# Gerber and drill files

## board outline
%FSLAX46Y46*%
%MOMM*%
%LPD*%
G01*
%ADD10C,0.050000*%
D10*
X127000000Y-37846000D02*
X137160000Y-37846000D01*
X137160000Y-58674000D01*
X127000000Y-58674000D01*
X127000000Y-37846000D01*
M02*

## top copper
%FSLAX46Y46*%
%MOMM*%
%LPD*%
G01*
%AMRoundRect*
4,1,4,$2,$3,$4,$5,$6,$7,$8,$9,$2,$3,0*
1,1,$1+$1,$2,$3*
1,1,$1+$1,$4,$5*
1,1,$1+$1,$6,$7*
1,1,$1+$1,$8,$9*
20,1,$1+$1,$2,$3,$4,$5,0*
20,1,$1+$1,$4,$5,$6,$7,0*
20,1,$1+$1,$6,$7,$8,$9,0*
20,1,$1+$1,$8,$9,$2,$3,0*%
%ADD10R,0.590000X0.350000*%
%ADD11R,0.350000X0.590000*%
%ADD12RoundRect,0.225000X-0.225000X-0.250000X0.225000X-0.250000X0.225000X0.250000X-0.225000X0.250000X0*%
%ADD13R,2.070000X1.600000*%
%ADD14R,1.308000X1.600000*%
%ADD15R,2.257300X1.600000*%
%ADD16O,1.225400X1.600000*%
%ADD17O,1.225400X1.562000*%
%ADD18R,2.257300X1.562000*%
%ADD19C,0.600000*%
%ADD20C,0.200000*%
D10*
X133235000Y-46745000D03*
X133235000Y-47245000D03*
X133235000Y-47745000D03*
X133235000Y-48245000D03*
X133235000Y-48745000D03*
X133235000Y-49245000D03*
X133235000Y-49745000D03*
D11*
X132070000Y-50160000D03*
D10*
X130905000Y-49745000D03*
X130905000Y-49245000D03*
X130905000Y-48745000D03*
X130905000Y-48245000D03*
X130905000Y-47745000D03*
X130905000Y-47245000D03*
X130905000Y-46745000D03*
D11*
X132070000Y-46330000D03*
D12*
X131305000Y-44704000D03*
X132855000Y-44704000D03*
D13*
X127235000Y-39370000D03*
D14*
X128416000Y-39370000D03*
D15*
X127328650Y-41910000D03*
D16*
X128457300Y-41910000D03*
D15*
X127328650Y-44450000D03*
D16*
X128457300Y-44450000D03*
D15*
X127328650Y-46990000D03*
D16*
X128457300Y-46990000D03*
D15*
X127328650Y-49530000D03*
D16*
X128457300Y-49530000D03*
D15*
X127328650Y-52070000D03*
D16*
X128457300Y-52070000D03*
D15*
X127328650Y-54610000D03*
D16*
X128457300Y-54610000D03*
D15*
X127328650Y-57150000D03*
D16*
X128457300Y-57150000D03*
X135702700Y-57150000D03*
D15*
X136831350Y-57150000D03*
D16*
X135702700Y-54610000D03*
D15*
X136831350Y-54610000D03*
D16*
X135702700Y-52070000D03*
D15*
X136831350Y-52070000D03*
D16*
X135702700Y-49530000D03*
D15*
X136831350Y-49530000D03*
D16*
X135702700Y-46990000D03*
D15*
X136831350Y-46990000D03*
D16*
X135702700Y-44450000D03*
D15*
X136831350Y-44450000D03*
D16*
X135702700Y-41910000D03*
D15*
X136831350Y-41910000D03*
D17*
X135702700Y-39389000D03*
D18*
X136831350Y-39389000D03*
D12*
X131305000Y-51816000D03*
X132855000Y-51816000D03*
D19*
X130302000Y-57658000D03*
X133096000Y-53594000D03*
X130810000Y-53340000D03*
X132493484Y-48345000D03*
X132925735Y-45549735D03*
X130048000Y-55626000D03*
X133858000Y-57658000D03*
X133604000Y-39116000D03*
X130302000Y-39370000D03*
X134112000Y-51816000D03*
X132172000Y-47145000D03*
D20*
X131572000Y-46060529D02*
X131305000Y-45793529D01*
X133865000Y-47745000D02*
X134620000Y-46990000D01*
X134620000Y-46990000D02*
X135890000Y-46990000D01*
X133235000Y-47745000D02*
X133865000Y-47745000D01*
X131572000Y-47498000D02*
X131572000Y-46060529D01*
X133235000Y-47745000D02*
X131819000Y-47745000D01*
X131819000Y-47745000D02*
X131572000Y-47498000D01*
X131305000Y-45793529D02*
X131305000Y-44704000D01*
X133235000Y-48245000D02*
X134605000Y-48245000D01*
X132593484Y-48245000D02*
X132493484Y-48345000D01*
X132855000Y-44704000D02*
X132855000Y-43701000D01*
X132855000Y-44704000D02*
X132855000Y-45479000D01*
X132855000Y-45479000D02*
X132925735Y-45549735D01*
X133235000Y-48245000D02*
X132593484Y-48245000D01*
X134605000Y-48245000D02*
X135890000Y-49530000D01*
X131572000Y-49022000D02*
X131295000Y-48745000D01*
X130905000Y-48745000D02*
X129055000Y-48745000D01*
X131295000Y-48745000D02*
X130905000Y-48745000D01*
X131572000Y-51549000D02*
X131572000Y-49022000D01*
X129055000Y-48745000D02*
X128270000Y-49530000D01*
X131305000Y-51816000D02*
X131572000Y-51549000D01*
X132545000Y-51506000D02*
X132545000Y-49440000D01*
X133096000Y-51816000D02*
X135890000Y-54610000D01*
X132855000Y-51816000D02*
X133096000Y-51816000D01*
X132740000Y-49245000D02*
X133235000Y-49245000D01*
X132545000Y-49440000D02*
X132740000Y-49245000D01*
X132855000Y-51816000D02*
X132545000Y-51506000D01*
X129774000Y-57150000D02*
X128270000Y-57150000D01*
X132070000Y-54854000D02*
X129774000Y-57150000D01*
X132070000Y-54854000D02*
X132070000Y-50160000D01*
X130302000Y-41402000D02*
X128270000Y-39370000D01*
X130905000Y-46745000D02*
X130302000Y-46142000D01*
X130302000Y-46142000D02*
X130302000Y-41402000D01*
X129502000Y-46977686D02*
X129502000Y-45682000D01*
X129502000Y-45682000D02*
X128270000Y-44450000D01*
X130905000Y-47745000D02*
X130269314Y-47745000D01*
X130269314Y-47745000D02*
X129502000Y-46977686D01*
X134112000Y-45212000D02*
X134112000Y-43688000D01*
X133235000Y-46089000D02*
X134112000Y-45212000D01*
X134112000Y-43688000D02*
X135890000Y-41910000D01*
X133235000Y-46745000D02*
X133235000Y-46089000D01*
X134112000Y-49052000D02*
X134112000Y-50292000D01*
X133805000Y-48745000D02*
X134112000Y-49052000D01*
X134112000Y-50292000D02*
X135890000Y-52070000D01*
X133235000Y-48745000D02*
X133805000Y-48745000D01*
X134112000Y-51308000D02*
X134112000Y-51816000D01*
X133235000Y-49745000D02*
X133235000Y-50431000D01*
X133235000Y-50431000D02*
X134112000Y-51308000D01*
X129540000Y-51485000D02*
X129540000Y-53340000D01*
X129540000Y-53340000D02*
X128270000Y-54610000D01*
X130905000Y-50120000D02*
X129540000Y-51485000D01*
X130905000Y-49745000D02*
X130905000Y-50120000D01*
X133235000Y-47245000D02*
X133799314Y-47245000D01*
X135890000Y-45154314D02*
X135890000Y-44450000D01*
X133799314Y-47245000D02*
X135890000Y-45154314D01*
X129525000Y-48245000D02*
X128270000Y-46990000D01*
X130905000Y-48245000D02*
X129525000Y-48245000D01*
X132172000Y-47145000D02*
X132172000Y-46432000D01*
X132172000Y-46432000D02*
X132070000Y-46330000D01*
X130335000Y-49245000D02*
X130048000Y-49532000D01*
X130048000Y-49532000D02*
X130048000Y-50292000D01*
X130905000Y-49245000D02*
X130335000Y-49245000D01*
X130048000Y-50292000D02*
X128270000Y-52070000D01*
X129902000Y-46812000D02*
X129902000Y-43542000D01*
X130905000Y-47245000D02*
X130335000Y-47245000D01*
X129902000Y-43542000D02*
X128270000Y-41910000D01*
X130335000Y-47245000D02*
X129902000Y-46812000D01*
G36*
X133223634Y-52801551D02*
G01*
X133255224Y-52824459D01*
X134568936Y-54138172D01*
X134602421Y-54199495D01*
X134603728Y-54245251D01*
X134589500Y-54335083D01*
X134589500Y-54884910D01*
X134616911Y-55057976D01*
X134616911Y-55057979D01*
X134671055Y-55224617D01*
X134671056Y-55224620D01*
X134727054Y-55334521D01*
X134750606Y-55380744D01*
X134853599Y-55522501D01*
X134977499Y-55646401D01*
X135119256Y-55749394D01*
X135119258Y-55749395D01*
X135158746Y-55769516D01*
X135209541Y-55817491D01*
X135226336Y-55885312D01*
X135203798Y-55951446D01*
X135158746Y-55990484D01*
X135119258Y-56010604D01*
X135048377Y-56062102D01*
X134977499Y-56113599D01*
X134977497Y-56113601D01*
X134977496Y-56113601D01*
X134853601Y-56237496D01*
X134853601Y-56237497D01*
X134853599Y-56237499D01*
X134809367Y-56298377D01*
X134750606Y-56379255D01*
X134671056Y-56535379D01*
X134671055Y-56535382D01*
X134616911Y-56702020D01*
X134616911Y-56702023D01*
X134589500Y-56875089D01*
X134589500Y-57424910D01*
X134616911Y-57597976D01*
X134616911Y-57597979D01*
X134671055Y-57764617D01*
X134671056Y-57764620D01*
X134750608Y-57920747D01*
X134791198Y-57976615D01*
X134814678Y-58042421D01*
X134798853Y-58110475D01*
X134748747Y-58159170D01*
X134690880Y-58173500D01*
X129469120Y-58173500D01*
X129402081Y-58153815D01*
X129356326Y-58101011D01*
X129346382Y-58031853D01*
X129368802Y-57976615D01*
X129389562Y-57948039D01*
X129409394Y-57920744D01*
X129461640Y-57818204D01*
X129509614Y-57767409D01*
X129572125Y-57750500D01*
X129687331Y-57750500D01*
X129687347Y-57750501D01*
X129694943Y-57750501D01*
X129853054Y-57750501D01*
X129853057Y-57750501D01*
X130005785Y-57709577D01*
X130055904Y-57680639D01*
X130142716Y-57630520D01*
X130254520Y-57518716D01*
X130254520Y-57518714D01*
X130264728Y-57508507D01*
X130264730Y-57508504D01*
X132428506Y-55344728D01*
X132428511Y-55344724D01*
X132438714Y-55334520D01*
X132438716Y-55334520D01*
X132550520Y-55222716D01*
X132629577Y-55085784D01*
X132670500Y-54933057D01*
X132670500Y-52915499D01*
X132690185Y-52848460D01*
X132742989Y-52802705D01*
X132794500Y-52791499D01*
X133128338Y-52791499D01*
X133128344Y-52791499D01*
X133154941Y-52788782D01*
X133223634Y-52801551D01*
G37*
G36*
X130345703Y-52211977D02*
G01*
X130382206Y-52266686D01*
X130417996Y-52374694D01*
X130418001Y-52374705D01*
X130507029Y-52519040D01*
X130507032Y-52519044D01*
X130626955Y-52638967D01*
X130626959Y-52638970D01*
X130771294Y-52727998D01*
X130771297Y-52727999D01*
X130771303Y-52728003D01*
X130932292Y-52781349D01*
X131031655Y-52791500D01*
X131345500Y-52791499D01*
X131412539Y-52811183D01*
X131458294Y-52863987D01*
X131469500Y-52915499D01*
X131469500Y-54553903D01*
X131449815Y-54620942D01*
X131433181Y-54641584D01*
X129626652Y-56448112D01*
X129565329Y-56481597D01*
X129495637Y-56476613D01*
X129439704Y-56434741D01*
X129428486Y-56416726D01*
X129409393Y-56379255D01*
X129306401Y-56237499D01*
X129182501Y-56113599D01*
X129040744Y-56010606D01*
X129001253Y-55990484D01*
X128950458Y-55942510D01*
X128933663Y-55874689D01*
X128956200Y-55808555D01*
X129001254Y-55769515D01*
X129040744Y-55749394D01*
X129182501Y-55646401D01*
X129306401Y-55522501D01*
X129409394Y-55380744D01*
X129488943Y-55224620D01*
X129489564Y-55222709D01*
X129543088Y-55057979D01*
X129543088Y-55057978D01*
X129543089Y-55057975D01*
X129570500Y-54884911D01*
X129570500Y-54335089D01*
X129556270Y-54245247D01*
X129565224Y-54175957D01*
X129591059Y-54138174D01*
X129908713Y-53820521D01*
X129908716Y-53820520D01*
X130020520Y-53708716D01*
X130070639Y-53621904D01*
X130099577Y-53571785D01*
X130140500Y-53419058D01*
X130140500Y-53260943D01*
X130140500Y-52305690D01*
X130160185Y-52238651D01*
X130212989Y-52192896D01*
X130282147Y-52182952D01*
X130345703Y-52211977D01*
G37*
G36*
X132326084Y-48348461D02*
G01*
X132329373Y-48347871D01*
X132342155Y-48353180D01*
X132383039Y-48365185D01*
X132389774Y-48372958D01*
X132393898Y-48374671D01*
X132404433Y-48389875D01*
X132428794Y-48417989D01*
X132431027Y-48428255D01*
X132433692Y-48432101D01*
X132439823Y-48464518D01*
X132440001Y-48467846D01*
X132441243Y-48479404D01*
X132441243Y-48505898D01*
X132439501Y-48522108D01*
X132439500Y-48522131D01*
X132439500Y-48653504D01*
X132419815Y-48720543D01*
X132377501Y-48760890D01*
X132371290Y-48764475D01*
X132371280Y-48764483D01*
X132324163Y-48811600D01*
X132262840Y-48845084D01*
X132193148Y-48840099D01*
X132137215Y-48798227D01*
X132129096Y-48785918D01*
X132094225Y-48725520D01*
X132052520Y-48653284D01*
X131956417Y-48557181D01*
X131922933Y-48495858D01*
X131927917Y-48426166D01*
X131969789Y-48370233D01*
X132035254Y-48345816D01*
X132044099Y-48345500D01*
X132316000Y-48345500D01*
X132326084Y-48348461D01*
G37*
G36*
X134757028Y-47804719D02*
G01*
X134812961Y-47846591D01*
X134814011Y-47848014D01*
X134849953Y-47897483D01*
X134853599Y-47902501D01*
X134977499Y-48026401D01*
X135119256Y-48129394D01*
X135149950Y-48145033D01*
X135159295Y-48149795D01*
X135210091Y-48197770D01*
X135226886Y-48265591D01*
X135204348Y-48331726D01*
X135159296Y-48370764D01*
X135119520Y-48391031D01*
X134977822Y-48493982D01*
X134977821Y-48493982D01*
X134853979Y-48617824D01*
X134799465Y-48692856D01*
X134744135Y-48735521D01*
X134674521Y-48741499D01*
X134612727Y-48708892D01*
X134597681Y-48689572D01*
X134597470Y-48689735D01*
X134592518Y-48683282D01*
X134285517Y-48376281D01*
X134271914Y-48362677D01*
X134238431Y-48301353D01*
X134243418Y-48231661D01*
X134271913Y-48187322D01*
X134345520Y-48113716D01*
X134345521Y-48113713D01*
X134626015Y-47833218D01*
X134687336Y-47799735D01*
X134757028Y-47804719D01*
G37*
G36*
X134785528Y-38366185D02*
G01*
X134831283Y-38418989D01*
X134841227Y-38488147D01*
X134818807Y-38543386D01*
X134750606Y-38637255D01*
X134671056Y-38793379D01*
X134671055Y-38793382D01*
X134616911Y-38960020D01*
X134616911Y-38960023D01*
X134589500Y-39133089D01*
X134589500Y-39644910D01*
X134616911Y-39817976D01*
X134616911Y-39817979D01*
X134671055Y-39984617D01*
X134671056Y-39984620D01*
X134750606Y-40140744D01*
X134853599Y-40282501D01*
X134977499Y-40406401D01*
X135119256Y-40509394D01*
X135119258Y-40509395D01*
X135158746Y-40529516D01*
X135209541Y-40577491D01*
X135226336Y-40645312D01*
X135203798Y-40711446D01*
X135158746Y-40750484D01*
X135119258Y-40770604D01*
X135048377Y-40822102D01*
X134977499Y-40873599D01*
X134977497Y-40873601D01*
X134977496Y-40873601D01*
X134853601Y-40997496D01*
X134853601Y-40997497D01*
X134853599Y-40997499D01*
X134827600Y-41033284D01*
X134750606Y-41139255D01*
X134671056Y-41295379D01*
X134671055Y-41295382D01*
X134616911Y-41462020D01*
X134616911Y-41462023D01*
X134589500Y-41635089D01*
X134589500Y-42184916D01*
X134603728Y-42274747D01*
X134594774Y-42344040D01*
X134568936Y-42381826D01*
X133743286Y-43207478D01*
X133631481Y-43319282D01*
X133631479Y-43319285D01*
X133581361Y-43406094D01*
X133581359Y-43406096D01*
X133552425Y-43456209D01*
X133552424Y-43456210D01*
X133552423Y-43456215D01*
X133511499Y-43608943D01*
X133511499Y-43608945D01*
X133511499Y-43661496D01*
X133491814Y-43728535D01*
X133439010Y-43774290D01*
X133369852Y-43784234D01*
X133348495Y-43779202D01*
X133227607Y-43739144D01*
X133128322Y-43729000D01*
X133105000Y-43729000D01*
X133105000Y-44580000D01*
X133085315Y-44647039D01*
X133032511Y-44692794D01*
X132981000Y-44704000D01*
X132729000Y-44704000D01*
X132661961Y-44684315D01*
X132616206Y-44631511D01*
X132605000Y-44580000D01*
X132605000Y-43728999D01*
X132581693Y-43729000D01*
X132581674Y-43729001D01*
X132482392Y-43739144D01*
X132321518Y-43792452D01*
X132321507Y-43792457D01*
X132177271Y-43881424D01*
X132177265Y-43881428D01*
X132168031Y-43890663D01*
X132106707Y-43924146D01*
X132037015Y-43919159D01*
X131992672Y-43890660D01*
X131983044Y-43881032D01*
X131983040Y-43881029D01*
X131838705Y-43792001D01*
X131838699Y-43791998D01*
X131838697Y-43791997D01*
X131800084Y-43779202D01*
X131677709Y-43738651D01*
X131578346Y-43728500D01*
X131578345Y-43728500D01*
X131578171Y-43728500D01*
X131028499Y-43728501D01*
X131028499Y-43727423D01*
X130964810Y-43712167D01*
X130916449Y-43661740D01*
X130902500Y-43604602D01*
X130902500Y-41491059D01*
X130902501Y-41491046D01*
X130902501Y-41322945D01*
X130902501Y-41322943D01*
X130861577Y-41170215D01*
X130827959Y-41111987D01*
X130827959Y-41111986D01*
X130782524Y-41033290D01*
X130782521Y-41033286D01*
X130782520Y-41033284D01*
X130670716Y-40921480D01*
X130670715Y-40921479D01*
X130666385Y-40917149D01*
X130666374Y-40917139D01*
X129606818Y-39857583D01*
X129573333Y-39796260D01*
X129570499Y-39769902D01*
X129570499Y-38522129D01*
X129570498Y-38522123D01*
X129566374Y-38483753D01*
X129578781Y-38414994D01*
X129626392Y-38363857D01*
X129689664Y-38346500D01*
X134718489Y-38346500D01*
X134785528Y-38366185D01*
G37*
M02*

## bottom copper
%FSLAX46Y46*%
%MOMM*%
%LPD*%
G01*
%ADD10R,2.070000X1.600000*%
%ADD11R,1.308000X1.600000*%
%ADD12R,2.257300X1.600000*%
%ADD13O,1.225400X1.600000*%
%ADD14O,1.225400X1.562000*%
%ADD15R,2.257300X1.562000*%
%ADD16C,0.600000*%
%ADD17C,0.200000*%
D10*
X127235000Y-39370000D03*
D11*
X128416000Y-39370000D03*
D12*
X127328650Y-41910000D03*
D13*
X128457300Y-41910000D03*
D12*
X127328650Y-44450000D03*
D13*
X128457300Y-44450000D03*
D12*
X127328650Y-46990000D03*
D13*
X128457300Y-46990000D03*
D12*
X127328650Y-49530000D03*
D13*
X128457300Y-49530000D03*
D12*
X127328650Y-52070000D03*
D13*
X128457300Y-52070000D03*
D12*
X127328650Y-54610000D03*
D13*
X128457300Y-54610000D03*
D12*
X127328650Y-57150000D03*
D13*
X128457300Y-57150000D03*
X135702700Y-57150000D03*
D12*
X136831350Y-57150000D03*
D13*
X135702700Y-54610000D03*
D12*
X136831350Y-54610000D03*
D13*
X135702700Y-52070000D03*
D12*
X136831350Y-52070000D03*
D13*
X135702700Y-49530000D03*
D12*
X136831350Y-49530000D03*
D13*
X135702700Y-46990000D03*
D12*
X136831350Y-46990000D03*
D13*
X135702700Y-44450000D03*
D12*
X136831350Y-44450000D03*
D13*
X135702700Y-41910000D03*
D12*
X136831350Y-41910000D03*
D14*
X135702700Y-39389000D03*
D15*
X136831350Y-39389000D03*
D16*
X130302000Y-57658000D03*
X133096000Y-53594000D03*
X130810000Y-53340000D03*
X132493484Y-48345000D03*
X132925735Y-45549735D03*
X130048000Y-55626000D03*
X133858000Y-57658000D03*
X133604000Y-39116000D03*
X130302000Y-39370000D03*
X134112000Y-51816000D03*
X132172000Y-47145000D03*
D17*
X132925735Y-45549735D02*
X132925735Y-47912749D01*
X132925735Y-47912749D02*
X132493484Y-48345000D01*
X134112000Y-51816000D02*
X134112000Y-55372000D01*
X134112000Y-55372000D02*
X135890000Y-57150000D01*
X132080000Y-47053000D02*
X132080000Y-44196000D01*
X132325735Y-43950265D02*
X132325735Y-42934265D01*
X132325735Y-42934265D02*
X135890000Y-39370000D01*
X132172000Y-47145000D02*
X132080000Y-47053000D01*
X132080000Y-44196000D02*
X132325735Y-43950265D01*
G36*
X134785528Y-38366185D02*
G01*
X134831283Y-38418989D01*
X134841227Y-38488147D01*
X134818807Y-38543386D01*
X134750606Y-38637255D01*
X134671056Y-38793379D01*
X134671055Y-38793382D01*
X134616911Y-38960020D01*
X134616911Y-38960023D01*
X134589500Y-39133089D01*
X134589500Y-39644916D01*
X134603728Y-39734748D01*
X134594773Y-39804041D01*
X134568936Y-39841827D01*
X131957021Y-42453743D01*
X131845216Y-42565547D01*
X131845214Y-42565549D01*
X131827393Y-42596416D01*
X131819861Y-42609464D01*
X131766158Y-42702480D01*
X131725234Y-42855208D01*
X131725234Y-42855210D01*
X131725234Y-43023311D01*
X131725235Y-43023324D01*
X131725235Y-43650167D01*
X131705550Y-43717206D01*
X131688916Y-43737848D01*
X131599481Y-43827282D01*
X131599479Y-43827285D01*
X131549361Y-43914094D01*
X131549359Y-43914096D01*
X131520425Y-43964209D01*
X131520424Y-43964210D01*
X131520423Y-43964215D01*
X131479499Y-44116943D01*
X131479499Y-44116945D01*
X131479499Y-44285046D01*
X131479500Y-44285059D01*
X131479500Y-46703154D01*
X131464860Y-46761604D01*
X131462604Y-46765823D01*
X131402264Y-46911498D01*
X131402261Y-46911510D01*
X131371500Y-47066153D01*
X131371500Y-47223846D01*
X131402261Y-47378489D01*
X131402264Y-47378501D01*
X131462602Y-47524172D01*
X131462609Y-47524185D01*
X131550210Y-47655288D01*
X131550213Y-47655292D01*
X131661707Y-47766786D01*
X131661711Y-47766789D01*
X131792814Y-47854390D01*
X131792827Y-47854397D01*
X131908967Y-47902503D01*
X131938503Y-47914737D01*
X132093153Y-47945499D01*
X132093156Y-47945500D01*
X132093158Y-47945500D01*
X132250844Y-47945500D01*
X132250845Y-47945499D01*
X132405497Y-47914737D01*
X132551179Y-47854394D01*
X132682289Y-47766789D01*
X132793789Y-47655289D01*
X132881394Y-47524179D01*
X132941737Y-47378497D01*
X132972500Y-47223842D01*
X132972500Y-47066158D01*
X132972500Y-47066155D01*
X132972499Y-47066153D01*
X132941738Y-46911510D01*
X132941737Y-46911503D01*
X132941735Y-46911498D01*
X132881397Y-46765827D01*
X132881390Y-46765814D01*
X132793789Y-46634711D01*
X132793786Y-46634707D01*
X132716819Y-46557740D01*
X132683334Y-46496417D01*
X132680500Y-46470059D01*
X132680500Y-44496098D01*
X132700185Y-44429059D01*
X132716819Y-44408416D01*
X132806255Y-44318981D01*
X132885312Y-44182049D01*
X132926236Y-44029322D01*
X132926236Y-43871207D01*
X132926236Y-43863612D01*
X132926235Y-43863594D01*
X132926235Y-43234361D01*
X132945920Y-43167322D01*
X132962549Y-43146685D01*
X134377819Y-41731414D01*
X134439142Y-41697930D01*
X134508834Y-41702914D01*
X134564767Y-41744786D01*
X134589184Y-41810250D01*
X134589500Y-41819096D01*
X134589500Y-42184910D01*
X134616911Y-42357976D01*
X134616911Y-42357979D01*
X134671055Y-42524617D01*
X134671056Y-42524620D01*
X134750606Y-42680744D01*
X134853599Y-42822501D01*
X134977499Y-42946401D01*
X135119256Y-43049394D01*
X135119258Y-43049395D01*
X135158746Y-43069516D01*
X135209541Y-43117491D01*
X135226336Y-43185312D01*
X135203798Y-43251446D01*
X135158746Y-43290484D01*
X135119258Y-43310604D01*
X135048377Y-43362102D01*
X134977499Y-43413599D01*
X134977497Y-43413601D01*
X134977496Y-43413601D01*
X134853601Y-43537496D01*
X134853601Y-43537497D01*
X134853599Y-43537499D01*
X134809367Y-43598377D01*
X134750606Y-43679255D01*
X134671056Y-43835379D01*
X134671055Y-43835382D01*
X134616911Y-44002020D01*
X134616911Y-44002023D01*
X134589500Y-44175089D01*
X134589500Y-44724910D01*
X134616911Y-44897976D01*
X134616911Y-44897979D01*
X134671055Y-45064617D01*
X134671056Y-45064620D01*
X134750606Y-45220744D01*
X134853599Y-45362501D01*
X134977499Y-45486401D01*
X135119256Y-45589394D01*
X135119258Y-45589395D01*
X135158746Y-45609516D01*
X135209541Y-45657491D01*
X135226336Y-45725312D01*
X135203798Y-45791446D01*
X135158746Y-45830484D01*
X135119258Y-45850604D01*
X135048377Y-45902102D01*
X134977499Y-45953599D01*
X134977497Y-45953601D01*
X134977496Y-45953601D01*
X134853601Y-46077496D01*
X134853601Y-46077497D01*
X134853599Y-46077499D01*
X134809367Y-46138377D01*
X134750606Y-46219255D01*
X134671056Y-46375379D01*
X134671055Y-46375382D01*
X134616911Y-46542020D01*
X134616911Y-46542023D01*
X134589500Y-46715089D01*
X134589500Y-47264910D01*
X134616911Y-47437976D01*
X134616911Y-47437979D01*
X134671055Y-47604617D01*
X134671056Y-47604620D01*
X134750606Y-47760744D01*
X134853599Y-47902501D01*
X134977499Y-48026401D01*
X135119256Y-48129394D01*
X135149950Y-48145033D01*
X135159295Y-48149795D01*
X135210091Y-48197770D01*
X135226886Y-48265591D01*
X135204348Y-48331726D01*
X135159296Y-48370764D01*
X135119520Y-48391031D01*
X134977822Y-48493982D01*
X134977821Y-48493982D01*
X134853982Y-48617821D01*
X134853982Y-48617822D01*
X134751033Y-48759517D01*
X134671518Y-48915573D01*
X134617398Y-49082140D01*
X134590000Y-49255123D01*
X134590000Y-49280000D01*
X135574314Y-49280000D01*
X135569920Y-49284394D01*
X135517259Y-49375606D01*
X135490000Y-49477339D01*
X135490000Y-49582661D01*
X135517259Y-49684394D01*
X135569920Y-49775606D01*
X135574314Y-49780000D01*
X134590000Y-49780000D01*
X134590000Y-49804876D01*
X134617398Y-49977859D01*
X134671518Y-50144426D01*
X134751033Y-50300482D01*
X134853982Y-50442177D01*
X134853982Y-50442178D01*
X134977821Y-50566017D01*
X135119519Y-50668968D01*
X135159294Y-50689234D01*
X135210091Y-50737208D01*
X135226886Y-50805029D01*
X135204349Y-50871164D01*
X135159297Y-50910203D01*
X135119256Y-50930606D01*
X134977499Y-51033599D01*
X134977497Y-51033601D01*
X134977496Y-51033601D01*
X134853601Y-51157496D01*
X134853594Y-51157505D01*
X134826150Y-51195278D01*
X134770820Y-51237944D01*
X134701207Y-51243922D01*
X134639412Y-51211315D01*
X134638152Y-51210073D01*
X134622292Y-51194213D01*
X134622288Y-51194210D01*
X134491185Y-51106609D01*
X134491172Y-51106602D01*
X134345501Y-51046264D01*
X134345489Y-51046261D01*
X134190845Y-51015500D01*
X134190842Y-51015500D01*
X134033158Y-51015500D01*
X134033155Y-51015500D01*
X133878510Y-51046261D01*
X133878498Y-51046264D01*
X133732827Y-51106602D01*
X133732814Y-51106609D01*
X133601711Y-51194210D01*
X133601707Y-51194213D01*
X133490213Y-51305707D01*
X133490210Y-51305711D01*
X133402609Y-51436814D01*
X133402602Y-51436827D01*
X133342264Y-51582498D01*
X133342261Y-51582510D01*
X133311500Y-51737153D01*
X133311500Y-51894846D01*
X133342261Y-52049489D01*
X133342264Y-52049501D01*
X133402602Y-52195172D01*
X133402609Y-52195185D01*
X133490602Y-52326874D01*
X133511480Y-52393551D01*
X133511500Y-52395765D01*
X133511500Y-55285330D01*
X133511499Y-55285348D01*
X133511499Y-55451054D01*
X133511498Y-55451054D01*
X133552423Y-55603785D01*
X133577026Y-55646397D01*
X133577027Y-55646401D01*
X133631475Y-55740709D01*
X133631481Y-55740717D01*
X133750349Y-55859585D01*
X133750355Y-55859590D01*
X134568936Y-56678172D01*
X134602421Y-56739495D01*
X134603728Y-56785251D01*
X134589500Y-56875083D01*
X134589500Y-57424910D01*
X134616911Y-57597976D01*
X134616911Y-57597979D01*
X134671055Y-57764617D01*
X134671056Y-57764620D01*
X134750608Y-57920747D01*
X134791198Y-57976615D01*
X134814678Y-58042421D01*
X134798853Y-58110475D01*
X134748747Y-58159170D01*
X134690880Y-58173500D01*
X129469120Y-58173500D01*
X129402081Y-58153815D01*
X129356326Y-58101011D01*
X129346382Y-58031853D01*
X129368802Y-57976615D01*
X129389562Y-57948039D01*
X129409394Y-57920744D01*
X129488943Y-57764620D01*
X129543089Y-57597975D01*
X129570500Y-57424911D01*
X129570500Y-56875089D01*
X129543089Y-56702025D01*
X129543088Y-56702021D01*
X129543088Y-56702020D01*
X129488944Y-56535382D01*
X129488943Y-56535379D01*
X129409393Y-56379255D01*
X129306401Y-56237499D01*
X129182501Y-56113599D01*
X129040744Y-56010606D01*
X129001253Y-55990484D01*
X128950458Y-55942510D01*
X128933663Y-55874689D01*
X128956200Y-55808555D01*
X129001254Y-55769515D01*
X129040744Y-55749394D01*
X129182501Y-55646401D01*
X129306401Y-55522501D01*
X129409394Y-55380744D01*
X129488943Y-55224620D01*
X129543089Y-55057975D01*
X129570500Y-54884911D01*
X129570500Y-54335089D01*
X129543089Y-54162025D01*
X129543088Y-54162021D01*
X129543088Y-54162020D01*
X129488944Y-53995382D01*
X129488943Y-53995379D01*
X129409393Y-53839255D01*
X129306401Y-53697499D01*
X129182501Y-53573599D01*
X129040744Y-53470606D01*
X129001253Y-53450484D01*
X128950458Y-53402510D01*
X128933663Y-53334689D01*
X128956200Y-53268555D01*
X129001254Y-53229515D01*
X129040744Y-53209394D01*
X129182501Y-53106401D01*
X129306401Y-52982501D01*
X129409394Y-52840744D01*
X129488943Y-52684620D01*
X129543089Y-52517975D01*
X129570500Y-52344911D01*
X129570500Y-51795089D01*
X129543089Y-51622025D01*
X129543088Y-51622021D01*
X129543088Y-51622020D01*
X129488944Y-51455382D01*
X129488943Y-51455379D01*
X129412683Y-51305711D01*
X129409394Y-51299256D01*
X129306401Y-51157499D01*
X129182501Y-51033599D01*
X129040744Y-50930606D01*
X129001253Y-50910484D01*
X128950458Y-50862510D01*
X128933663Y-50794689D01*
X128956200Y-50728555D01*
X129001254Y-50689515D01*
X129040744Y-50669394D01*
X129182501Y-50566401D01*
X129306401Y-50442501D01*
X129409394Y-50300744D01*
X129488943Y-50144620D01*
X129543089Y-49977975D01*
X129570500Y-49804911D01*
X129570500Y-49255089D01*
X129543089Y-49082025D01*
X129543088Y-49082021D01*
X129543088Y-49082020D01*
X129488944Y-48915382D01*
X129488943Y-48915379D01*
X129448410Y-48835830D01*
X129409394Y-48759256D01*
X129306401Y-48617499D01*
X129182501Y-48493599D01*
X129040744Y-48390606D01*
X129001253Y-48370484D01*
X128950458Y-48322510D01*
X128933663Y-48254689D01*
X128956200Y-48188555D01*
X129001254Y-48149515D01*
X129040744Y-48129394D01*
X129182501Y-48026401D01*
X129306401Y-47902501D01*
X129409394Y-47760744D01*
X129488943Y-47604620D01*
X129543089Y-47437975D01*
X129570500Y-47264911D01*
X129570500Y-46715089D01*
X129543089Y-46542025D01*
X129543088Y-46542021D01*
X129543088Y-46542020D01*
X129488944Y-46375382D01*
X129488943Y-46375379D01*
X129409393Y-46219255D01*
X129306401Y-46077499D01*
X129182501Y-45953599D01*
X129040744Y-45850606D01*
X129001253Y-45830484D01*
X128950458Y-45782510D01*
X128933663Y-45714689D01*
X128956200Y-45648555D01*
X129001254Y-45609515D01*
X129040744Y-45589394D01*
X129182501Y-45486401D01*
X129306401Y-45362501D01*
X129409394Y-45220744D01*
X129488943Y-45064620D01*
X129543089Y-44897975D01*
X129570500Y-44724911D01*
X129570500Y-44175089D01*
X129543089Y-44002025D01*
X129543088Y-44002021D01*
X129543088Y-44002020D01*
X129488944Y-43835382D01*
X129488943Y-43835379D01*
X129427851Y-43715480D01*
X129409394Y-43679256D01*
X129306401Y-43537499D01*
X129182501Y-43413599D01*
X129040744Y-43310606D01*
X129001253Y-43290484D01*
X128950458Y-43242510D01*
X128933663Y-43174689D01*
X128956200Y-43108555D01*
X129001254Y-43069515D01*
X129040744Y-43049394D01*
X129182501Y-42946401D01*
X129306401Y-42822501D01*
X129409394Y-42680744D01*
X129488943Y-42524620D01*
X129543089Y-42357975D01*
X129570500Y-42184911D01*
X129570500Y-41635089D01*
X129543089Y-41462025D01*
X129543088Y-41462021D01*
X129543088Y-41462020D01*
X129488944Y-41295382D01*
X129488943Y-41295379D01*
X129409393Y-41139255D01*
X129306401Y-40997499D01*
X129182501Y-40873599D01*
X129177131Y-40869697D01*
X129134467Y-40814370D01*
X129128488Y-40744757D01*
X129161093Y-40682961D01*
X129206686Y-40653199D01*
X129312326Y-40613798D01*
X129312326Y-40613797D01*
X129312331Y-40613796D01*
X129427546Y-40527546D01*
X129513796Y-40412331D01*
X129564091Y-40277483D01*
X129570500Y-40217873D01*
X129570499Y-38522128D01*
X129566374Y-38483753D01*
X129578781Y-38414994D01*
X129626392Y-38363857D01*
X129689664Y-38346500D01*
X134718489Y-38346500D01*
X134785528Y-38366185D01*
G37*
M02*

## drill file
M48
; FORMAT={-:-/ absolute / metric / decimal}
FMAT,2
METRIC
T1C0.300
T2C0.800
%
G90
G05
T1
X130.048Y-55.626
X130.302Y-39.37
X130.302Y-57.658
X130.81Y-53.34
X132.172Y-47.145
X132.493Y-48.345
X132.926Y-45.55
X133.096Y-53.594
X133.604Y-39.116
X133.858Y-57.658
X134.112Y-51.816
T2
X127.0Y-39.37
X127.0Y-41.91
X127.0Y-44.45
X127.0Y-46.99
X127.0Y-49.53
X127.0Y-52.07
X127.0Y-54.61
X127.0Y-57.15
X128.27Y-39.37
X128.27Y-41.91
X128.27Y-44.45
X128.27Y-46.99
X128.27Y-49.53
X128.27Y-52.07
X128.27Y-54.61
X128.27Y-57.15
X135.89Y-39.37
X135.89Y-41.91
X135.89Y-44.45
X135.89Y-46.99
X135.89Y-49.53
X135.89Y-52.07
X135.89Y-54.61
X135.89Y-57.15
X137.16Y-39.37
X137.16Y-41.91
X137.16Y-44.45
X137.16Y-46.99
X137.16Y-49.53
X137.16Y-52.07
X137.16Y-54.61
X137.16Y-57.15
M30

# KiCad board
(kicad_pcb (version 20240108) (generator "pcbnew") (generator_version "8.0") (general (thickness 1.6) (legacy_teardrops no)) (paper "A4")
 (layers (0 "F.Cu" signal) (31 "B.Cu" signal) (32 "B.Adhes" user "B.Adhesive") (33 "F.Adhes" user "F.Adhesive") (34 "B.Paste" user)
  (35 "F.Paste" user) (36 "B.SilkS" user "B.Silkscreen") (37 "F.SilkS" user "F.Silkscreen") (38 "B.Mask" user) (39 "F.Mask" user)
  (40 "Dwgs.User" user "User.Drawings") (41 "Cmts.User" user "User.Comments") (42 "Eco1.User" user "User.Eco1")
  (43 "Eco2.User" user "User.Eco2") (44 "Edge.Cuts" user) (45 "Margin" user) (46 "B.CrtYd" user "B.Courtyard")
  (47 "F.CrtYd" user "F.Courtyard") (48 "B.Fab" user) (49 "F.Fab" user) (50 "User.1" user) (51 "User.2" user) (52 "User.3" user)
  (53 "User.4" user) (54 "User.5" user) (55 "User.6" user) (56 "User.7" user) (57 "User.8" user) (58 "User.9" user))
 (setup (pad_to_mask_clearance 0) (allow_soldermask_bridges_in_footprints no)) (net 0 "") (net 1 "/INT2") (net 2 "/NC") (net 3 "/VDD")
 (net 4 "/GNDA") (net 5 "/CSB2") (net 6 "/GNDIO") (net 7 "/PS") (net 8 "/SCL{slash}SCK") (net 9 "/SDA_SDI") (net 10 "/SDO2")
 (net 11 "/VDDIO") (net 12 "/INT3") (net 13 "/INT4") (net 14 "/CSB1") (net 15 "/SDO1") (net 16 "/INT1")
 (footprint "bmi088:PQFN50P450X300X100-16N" (layer "F.Cu") (at 132.07 48.245 -90)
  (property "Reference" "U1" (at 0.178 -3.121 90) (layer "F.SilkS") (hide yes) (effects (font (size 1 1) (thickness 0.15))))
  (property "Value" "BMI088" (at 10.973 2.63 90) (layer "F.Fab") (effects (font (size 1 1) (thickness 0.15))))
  (pad "1" smd rect (at -1.5 -1.165 270) (size 0.35 0.59) (layers "F.Cu" "F.Paste" "F.Mask") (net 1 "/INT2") (solder_mask_margin 0.03))
  (pad "2" smd rect (at -1 -1.165 270) (size 0.35 0.59) (layers "F.Cu" "F.Paste" "F.Mask") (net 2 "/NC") (solder_mask_margin 0.03))
  (pad "3" smd rect (at -0.5 -1.165 270) (size 0.35 0.59) (layers "F.Cu" "F.Paste" "F.Mask") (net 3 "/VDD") (solder_mask_margin 0.03))
  (pad "4" smd rect (at 0 -1.165 270) (size 0.35 0.59) (layers "F.Cu" "F.Paste" "F.Mask") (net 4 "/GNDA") (solder_mask_margin 0.03))
  (pad "5" smd rect (at 0.5 -1.165 270) (size 0.35 0.59) (layers "F.Cu" "F.Paste" "F.Mask") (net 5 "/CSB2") (solder_mask_margin 0.03))
  (pad "6" smd rect (at 1 -1.165 270) (size 0.35 0.59) (layers "F.Cu" "F.Paste" "F.Mask") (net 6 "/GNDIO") (solder_mask_margin 0.03))
  (pad "7" smd rect (at 1.5 -1.165 270) (size 0.35 0.59) (layers "F.Cu" "F.Paste" "F.Mask") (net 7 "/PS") (solder_mask_margin 0.03))
  (pad "8" smd rect (at 1.915 0 270) (size 0.59 0.35) (layers "F.Cu" "F.Paste" "F.Mask") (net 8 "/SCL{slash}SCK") (solder_mask_margin 0.03))
  (pad "9" smd rect (at 1.5 1.165 270) (size 0.35 0.59) (layers "F.Cu" "F.Paste" "F.Mask") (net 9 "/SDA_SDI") (solder_mask_margin 0.03))
  (pad "10" smd rect (at 1 1.165 270) (size 0.35 0.59) (layers "F.Cu" "F.Paste" "F.Mask") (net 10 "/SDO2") (solder_mask_margin 0.03))
  (pad "11" smd rect (at 0.5 1.165 270) (size 0.35 0.59) (layers "F.Cu" "F.Paste" "F.Mask") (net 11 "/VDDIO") (solder_mask_margin 0.03))
  (pad "12" smd rect (at 0 1.165 270) (size 0.35 0.59) (layers "F.Cu" "F.Paste" "F.Mask") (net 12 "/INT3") (solder_mask_margin 0.03))
  (pad "13" smd rect (at -0.5 1.165 270) (size 0.35 0.59) (layers "F.Cu" "F.Paste" "F.Mask") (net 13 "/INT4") (solder_mask_margin 0.03))
  (pad "14" smd rect (at -1 1.165 270) (size 0.35 0.59) (layers "F.Cu" "F.Paste" "F.Mask") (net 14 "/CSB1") (solder_mask_margin 0.03))
  (pad "15" smd rect (at -1.5 1.165 270) (size 0.35 0.59) (layers "F.Cu" "F.Paste" "F.Mask") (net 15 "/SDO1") (solder_mask_margin 0.03))
  (pad "16" smd rect (at -1.915 0 270) (size 0.59 0.35) (layers "F.Cu" "F.Paste" "F.Mask") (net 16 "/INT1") (solder_mask_margin 0.03)))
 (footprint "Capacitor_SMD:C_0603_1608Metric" (layer "F.Cu") (at 132.08 44.704)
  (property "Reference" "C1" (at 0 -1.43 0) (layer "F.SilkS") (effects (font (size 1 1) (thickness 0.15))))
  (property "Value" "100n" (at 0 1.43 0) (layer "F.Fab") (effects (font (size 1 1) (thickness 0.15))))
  (pad "1" smd roundrect (at -0.775 0) (size 0.9 0.95) (layers "F.Cu" "F.Paste" "F.Mask") (roundrect_rratio 0.25) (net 3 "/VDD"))
  (pad "2" smd roundrect (at 0.775 0) (size 0.9 0.95) (layers "F.Cu" "F.Paste" "F.Mask") (roundrect_rratio 0.25) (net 4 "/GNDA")))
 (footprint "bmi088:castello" (layer "F.Cu") (at 128.27 39.37)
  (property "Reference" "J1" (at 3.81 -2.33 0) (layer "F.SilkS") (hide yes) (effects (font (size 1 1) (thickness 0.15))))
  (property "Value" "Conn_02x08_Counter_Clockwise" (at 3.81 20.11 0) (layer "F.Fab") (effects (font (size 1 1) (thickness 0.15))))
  (pad "1" thru_hole rect (at -1.27 0) (size 2.07 1.6) (drill 0.8 (offset 0.235 0)) (layers "*.Cu" "*.Mask") (remove_unused_layers no)
   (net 15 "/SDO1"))
  (pad "1" thru_hole rect (at 0 0) (size 1.308 1.6) (drill 0.8 (offset 0.146 0)) (layers "*.Cu" "*.Mask") (remove_unused_layers no)
   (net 15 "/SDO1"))
  (pad "2" thru_hole rect (at -1.27 2.54) (size 2.2573 1.6) (drill 0.8 (offset 0.32865 0)) (layers "*.Cu" "*.Mask")
   (remove_unused_layers no) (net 14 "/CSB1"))
  (pad "2" thru_hole oval (at 0 2.54) (size 1.2254 1.6) (drill 0.8 (offset 0.1873 0)) (layers "*.Cu" "*.Mask") (remove_unused_layers no)
   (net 14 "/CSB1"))
  (pad "3" thru_hole rect (at -1.27 5.08) (size 2.2573 1.6) (drill 0.8 (offset 0.32865 0)) (layers "*.Cu" "*.Mask")
   (remove_unused_layers no) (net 13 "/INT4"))
  (pad "3" thru_hole oval (at 0 5.08) (size 1.2254 1.6) (drill 0.8 (offset 0.1873 0)) (layers "*.Cu" "*.Mask") (remove_unused_layers no)
   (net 13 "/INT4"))
  (pad "4" thru_hole rect (at -1.27 7.62) (size 2.2573 1.6) (drill 0.8 (offset 0.32865 0)) (layers "*.Cu" "*.Mask")
   (remove_unused_layers no) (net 12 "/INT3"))
  (pad "4" thru_hole oval (at 0 7.62) (size 1.2254 1.6) (drill 0.8 (offset 0.1873 0)) (layers "*.Cu" "*.Mask") (remove_unused_layers no)
   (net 12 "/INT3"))
  (pad "5" thru_hole rect (at -1.27 10.16) (size 2.2573 1.6) (drill 0.8 (offset 0.32865 0)) (layers "*.Cu" "*.Mask")
   (remove_unused_layers no) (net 11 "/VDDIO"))
  (pad "5" thru_hole oval (at 0 10.16) (size 1.2254 1.6) (drill 0.8 (offset 0.1873 0)) (layers "*.Cu" "*.Mask") (remove_unused_layers no)
   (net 11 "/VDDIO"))
  (pad "6" thru_hole rect (at -1.27 12.7 180) (size 2.2573 1.6) (drill 0.8 (offset -0.32865 0)) (layers "*.Cu" "*.Mask")
   (remove_unused_layers no) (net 10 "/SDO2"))
  (pad "6" thru_hole oval (at 0 12.7) (size 1.2254 1.6) (drill 0.8 (offset 0.1873 0)) (layers "*.Cu" "*.Mask") (remove_unused_layers no)
   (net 10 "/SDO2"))
  (pad "7" thru_hole rect (at -1.27 15.24) (size 2.2573 1.6) (drill 0.8 (offset 0.32865 0)) (layers "*.Cu" "*.Mask")
   (remove_unused_layers no) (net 9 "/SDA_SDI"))
  (pad "7" thru_hole oval (at 0 15.24) (size 1.2254 1.6) (drill 0.8 (offset 0.1873 0)) (layers "*.Cu" "*.Mask") (remove_unused_layers no)
   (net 9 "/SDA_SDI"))
  (pad "8" thru_hole rect (at -1.27 17.78) (size 2.2573 1.6) (drill 0.8 (offset 0.32865 0)) (layers "*.Cu" "*.Mask")
   (remove_unused_layers no) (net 8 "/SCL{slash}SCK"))
  (pad "8" thru_hole oval (at 0 17.78) (size 1.2254 1.6) (drill 0.8 (offset 0.1873 0)) (layers "*.Cu" "*.Mask") (remove_unused_layers no)
   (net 8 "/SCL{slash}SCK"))
  (pad "9" thru_hole oval (at 7.62 17.78) (size 1.2254 1.6) (drill 0.8 (offset -0.1873 0)) (layers "*.Cu" "*.Mask")
   (remove_unused_layers no) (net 7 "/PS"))
  (pad "9" thru_hole rect (at 8.89 17.78) (size 2.2573 1.6) (drill 0.8 (offset -0.32865 0)) (layers "*.Cu" "*.Mask")
   (remove_unused_layers no) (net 7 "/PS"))
  (pad "10" thru_hole oval (at 7.62 15.24) (size 1.2254 1.6) (drill 0.8 (offset -0.1873 0)) (layers "*.Cu" "*.Mask")
   (remove_unused_layers no) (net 6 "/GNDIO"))
  (pad "10" thru_hole rect (at 8.89 15.24) (size 2.2573 1.6) (drill 0.8 (offset -0.32865 0)) (layers "*.Cu" "*.Mask")
   (remove_unused_layers no) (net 6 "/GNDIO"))
  (pad "11" thru_hole oval (at 7.62 12.7) (size 1.2254 1.6) (drill 0.8 (offset -0.1873 0)) (layers "*.Cu" "*.Mask")
   (remove_unused_layers no) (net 5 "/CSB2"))
  (pad "11" thru_hole rect (at 8.89 12.7) (size 2.2573 1.6) (drill 0.8 (offset -0.32865 0)) (layers "*.Cu" "*.Mask")
   (remove_unused_layers no) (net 5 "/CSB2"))
  (pad "12" thru_hole oval (at 7.62 10.16) (size 1.2254 1.6) (drill 0.8 (offset -0.1873 0)) (layers "*.Cu" "*.Mask")
   (remove_unused_layers no) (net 4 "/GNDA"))
  (pad "12" thru_hole rect (at 8.89 10.16) (size 2.2573 1.6) (drill 0.8 (offset -0.32865 0)) (layers "*.Cu" "*.Mask")
   (remove_unused_layers no) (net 4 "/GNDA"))
  (pad "13" thru_hole oval (at 7.62 7.62) (size 1.2254 1.6) (drill 0.8 (offset -0.1873 0)) (layers "*.Cu" "*.Mask")
   (remove_unused_layers no) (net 3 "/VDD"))
  (pad "13" thru_hole rect (at 8.89 7.62) (size 2.2573 1.6) (drill 0.8 (offset -0.32865 0)) (layers "*.Cu" "*.Mask")
   (remove_unused_layers no) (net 3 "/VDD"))
  (pad "14" thru_hole oval (at 7.62 5.08) (size 1.2254 1.6) (drill 0.8 (offset -0.1873 0)) (layers "*.Cu" "*.Mask")
   (remove_unused_layers no) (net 2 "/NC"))
  (pad "14" thru_hole rect (at 8.89 5.08) (size 2.2573 1.6) (drill 0.8 (offset -0.32865 0)) (layers "*.Cu" "*.Mask")
   (remove_unused_layers no) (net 2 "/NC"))
  (pad "15" thru_hole oval (at 7.62 2.54) (size 1.2254 1.6) (drill 0.8 (offset -0.1873 0)) (layers "*.Cu" "*.Mask")
   (remove_unused_layers no) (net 1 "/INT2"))
  (pad "15" thru_hole rect (at 8.89 2.54) (size 2.2573 1.6) (drill 0.8 (offset -0.32865 0)) (layers "*.Cu" "*.Mask")
   (remove_unused_layers no) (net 1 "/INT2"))
  (pad "16" thru_hole oval (at 7.62 0) (size 1.2254 1.562) (drill 0.8 (offset -0.1873 0.019)) (layers "*.Cu" "*.Mask")
   (remove_unused_layers no) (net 16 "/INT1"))
  (pad "16" thru_hole rect (at 8.89 0) (size 2.2573 1.562) (drill 0.8 (offset -0.32865 0.019)) (layers "*.Cu" "*.Mask")
   (remove_unused_layers no) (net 16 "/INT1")))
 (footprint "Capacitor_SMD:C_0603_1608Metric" (layer "F.Cu") (at 132.08 51.816)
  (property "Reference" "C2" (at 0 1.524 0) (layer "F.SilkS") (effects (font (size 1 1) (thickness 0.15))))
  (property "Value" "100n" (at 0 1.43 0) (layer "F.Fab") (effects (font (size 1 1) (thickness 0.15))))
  (pad "1" smd roundrect (at -0.775 0) (size 0.9 0.95) (layers "F.Cu" "F.Paste" "F.Mask") (roundrect_rratio 0.25) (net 11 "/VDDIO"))
  (pad "2" smd roundrect (at 0.775 0) (size 0.9 0.95) (layers "F.Cu" "F.Paste" "F.Mask") (roundrect_rratio 0.25) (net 6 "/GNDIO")))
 (gr_rect (start 127 37.846) (end 137.16 58.674) (stroke (width 0.05) (type default)) (fill none) (layer "Edge.Cuts"))
 (segment (start 131.572 46.060529) (end 131.305 45.793529) (width 0.2) (layer "F.Cu") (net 3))
 (segment (start 133.865 47.745) (end 134.62 46.99) (width 0.2) (layer "F.Cu") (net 3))
 (segment (start 134.62 46.99) (end 135.89 46.99) (width 0.2) (layer "F.Cu") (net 3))
 (segment (start 133.235 47.745) (end 133.865 47.745) (width 0.2) (layer "F.Cu") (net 3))
 (segment (start 131.572 47.498) (end 131.572 46.060529) (width 0.2) (layer "F.Cu") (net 3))
 (segment (start 133.235 47.745) (end 131.819 47.745) (width 0.2) (layer "F.Cu") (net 3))
 (segment (start 131.819 47.745) (end 131.572 47.498) (width 0.2) (layer "F.Cu") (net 3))
 (segment (start 131.305 45.793529) (end 131.305 44.704) (width 0.2) (layer "F.Cu") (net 3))
 (segment (start 133.235 48.245) (end 134.605 48.245) (width 0.2) (layer "F.Cu") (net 4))
 (segment (start 132.593484 48.245) (end 132.493484 48.345) (width 0.2) (layer "F.Cu") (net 4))
 (segment (start 132.855 44.704) (end 132.855 43.701) (width 0.2) (layer "F.Cu") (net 4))
 (segment (start 132.855 44.704) (end 132.855 45.479) (width 0.2) (layer "F.Cu") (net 4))
 (segment (start 132.855 45.479) (end 132.925735 45.549735) (width 0.2) (layer "F.Cu") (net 4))
 (segment (start 133.235 48.245) (end 132.593484 48.245) (width 0.2) (layer "F.Cu") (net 4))
 (segment (start 134.605 48.245) (end 135.89 49.53) (width 0.2) (layer "F.Cu") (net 4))
 (via (at 130.302 57.658) (size 0.6) (drill 0.3) (layers "F.Cu" "B.Cu") (free yes) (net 4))
 (via (at 133.096 53.594) (size 0.6) (drill 0.3) (layers "F.Cu" "B.Cu") (free yes) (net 4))
 (via (at 130.81 53.34) (size 0.6) (drill 0.3) (layers "F.Cu" "B.Cu") (free yes) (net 4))
 (via (at 132.493484 48.345) (size 0.6) (drill 0.3) (layers "F.Cu" "B.Cu") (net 4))
 (via (at 132.925735 45.549735) (size 0.6) (drill 0.3) (layers "F.Cu" "B.Cu") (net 4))
 (via (at 130.048 55.626) (size 0.6) (drill 0.3) (layers "F.Cu" "B.Cu") (free yes) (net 4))
 (via (at 133.858 57.658) (size 0.6) (drill 0.3) (layers "F.Cu" "B.Cu") (free yes) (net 4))
 (via (at 133.604 39.116) (size 0.6) (drill 0.3) (layers "F.Cu" "B.Cu") (free yes) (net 4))
 (via (at 130.302 39.37) (size 0.6) (drill 0.3) (layers "F.Cu" "B.Cu") (free yes) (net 4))
 (segment (start 132.925735 45.549735) (end 132.925735 47.912749) (width 0.2) (layer "B.Cu") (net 4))
 (segment (start 132.925735 47.912749) (end 132.493484 48.345) (width 0.2) (layer "B.Cu") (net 4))
 (segment (start 131.572 49.022) (end 131.295 48.745) (width 0.2) (layer "F.Cu") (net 11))
 (segment (start 130.905 48.745) (end 129.055 48.745) (width 0.2) (layer "F.Cu") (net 11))
 (segment (start 131.295 48.745) (end 130.905 48.745) (width 0.2) (layer "F.Cu") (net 11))
 (segment (start 131.572 51.549) (end 131.572 49.022) (width 0.2) (layer "F.Cu") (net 11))
 (segment (start 129.055 48.745) (end 128.27 49.53) (width 0.2) (layer "F.Cu") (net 11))
 (segment (start 131.305 51.816) (end 131.572 51.549) (width 0.2) (layer "F.Cu") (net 11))
 (segment (start 132.545 51.506) (end 132.545 49.44) (width 0.2) (layer "F.Cu") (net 6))
 (segment (start 133.096 51.816) (end 135.89 54.61) (width 0.2) (layer "F.Cu") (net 6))
 (segment (start 132.855 51.816) (end 133.096 51.816) (width 0.2) (layer "F.Cu") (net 6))
 (segment (start 132.74 49.245) (end 133.235 49.245) (width 0.2) (layer "F.Cu") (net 6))
 (segment (start 132.545 49.44) (end 132.74 49.245) (width 0.2) (layer "F.Cu") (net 6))
 (segment (start 132.855 51.816) (end 132.545 51.506) (width 0.2) (layer "F.Cu") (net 6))
 (segment (start 129.774 57.15) (end 128.27 57.15) (width 0.2) (layer "F.Cu") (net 8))
 (segment (start 132.07 54.854) (end 129.774 57.15) (width 0.2) (layer "F.Cu") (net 8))
 (segment (start 132.07 54.854) (end 132.07 50.16) (width 0.2) (layer "F.Cu") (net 8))
 (segment (start 130.302 41.402) (end 128.27 39.37) (width 0.2) (layer "F.Cu") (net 15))
 (segment (start 130.905 46.745) (end 130.302 46.142) (width 0.2) (layer "F.Cu") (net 15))
 (segment (start 130.302 46.142) (end 130.302 41.402) (width 0.2) (layer "F.Cu") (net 15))
 (segment (start 129.502 46.977686) (end 129.502 45.682) (width 0.2) (layer "F.Cu") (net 13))
 (segment (start 129.502 45.682) (end 128.27 44.45) (width 0.2) (layer "F.Cu") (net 13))
 (segment (start 130.905 47.745) (end 130.269314 47.745) (width 0.2) (layer "F.Cu") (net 13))
 (segment (start 130.269314 47.745) (end 129.502 46.977686) (width 0.2) (layer "F.Cu") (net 13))
 (segment (start 134.112 45.212) (end 134.112 43.688) (width 0.2) (layer "F.Cu") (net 1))
 (segment (start 133.235 46.089) (end 134.112 45.212) (width 0.2) (layer "F.Cu") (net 1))
 (segment (start 134.112 43.688) (end 135.89 41.91) (width 0.2) (layer "F.Cu") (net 1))
 (segment (start 133.235 46.745) (end 133.235 46.089) (width 0.2) (layer "F.Cu") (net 1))
 (segment (start 134.112 49.052) (end 134.112 50.292) (width 0.2) (layer "F.Cu") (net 5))
 (segment (start 133.805 48.745) (end 134.112 49.052) (width 0.2) (layer "F.Cu") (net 5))
 (segment (start 134.112 50.292) (end 135.89 52.07) (width 0.2) (layer "F.Cu") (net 5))
 (segment (start 133.235 48.745) (end 133.805 48.745) (width 0.2) (layer "F.Cu") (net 5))
 (segment (start 134.112 51.308) (end 134.112 51.816) (width 0.2) (layer "F.Cu") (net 7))
 (segment (start 133.235 49.745) (end 133.235 50.431) (width 0.2) (layer "F.Cu") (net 7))
 (segment (start 133.235 50.431) (end 134.112 51.308) (width 0.2) (layer "F.Cu") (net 7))
 (via (at 134.112 51.816) (size 0.6) (drill 0.3) (layers "F.Cu" "B.Cu") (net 7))
 (segment (start 134.112 51.816) (end 134.112 55.372) (width 0.2) (layer "B.Cu") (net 7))
 (segment (start 134.112 55.372) (end 135.89 57.15) (width 0.2) (layer "B.Cu") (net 7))
 (segment (start 129.54 51.485) (end 129.54 53.34) (width 0.2) (layer "F.Cu") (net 9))
 (segment (start 129.54 53.34) (end 128.27 54.61) (width 0.2) (layer "F.Cu") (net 9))
 (segment (start 130.905 50.12) (end 129.54 51.485) (width 0.2) (layer "F.Cu") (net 9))
 (segment (start 130.905 49.745) (end 130.905 50.12) (width 0.2) (layer "F.Cu") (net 9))
 (segment (start 133.235 47.245) (end 133.799314 47.245) (width 0.2) (layer "F.Cu") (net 2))
 (segment (start 135.89 45.154314) (end 135.89 44.45) (width 0.2) (layer "F.Cu") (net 2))
 (segment (start 133.799314 47.245) (end 135.89 45.154314) (width 0.2) (layer "F.Cu") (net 2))
 (segment (start 129.525 48.245) (end 128.27 46.99) (width 0.2) (layer "F.Cu") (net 12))
 (segment (start 130.905 48.245) (end 129.525 48.245) (width 0.2) (layer "F.Cu") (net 12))
 (segment (start 132.172 47.145) (end 132.172 46.432) (width 0.2) (layer "F.Cu") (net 16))
 (segment (start 132.172 46.432) (end 132.07 46.33) (width 0.2) (layer "F.Cu") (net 16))
 (via (at 132.172 47.145) (size 0.6) (drill 0.3) (layers "F.Cu" "B.Cu") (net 16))
 (segment (start 132.08 47.053) (end 132.08 44.196) (width 0.2) (layer "B.Cu") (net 16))
 (segment (start 132.325735 43.950265) (end 132.325735 42.934265) (width 0.2) (layer "B.Cu") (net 16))
 (segment (start 132.325735 42.934265) (end 135.89 39.37) (width 0.2) (layer "B.Cu") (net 16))
 (segment (start 132.172 47.145) (end 132.08 47.053) (width 0.2) (layer "B.Cu") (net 16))
 (segment (start 132.08 44.196) (end 132.325735 43.950265) (width 0.2) (layer "B.Cu") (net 16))
 (segment (start 130.335 49.245) (end 130.048 49.532) (width 0.2) (layer "F.Cu") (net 10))
 (segment (start 130.048 49.532) (end 130.048 50.292) (width 0.2) (layer "F.Cu") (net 10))
 (segment (start 130.905 49.245) (end 130.335 49.245) (width 0.2) (layer "F.Cu") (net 10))
 (segment (start 130.048 50.292) (end 128.27 52.07) (width 0.2) (layer "F.Cu") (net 10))
 (segment (start 129.902 46.812) (end 129.902 43.542) (width 0.2) (layer "F.Cu") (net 14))
 (segment (start 130.905 47.245) (end 130.335 47.245) (width 0.2) (layer "F.Cu") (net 14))
 (segment (start 129.902 43.542) (end 128.27 41.91) (width 0.2) (layer "F.Cu") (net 14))
 (segment (start 130.335 47.245) (end 129.902 46.812) (width 0.2) (layer "F.Cu") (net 14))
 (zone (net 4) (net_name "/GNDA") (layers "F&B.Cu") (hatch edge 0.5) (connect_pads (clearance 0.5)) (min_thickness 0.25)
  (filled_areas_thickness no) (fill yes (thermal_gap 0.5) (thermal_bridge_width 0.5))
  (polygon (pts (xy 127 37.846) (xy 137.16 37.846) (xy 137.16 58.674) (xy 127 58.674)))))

